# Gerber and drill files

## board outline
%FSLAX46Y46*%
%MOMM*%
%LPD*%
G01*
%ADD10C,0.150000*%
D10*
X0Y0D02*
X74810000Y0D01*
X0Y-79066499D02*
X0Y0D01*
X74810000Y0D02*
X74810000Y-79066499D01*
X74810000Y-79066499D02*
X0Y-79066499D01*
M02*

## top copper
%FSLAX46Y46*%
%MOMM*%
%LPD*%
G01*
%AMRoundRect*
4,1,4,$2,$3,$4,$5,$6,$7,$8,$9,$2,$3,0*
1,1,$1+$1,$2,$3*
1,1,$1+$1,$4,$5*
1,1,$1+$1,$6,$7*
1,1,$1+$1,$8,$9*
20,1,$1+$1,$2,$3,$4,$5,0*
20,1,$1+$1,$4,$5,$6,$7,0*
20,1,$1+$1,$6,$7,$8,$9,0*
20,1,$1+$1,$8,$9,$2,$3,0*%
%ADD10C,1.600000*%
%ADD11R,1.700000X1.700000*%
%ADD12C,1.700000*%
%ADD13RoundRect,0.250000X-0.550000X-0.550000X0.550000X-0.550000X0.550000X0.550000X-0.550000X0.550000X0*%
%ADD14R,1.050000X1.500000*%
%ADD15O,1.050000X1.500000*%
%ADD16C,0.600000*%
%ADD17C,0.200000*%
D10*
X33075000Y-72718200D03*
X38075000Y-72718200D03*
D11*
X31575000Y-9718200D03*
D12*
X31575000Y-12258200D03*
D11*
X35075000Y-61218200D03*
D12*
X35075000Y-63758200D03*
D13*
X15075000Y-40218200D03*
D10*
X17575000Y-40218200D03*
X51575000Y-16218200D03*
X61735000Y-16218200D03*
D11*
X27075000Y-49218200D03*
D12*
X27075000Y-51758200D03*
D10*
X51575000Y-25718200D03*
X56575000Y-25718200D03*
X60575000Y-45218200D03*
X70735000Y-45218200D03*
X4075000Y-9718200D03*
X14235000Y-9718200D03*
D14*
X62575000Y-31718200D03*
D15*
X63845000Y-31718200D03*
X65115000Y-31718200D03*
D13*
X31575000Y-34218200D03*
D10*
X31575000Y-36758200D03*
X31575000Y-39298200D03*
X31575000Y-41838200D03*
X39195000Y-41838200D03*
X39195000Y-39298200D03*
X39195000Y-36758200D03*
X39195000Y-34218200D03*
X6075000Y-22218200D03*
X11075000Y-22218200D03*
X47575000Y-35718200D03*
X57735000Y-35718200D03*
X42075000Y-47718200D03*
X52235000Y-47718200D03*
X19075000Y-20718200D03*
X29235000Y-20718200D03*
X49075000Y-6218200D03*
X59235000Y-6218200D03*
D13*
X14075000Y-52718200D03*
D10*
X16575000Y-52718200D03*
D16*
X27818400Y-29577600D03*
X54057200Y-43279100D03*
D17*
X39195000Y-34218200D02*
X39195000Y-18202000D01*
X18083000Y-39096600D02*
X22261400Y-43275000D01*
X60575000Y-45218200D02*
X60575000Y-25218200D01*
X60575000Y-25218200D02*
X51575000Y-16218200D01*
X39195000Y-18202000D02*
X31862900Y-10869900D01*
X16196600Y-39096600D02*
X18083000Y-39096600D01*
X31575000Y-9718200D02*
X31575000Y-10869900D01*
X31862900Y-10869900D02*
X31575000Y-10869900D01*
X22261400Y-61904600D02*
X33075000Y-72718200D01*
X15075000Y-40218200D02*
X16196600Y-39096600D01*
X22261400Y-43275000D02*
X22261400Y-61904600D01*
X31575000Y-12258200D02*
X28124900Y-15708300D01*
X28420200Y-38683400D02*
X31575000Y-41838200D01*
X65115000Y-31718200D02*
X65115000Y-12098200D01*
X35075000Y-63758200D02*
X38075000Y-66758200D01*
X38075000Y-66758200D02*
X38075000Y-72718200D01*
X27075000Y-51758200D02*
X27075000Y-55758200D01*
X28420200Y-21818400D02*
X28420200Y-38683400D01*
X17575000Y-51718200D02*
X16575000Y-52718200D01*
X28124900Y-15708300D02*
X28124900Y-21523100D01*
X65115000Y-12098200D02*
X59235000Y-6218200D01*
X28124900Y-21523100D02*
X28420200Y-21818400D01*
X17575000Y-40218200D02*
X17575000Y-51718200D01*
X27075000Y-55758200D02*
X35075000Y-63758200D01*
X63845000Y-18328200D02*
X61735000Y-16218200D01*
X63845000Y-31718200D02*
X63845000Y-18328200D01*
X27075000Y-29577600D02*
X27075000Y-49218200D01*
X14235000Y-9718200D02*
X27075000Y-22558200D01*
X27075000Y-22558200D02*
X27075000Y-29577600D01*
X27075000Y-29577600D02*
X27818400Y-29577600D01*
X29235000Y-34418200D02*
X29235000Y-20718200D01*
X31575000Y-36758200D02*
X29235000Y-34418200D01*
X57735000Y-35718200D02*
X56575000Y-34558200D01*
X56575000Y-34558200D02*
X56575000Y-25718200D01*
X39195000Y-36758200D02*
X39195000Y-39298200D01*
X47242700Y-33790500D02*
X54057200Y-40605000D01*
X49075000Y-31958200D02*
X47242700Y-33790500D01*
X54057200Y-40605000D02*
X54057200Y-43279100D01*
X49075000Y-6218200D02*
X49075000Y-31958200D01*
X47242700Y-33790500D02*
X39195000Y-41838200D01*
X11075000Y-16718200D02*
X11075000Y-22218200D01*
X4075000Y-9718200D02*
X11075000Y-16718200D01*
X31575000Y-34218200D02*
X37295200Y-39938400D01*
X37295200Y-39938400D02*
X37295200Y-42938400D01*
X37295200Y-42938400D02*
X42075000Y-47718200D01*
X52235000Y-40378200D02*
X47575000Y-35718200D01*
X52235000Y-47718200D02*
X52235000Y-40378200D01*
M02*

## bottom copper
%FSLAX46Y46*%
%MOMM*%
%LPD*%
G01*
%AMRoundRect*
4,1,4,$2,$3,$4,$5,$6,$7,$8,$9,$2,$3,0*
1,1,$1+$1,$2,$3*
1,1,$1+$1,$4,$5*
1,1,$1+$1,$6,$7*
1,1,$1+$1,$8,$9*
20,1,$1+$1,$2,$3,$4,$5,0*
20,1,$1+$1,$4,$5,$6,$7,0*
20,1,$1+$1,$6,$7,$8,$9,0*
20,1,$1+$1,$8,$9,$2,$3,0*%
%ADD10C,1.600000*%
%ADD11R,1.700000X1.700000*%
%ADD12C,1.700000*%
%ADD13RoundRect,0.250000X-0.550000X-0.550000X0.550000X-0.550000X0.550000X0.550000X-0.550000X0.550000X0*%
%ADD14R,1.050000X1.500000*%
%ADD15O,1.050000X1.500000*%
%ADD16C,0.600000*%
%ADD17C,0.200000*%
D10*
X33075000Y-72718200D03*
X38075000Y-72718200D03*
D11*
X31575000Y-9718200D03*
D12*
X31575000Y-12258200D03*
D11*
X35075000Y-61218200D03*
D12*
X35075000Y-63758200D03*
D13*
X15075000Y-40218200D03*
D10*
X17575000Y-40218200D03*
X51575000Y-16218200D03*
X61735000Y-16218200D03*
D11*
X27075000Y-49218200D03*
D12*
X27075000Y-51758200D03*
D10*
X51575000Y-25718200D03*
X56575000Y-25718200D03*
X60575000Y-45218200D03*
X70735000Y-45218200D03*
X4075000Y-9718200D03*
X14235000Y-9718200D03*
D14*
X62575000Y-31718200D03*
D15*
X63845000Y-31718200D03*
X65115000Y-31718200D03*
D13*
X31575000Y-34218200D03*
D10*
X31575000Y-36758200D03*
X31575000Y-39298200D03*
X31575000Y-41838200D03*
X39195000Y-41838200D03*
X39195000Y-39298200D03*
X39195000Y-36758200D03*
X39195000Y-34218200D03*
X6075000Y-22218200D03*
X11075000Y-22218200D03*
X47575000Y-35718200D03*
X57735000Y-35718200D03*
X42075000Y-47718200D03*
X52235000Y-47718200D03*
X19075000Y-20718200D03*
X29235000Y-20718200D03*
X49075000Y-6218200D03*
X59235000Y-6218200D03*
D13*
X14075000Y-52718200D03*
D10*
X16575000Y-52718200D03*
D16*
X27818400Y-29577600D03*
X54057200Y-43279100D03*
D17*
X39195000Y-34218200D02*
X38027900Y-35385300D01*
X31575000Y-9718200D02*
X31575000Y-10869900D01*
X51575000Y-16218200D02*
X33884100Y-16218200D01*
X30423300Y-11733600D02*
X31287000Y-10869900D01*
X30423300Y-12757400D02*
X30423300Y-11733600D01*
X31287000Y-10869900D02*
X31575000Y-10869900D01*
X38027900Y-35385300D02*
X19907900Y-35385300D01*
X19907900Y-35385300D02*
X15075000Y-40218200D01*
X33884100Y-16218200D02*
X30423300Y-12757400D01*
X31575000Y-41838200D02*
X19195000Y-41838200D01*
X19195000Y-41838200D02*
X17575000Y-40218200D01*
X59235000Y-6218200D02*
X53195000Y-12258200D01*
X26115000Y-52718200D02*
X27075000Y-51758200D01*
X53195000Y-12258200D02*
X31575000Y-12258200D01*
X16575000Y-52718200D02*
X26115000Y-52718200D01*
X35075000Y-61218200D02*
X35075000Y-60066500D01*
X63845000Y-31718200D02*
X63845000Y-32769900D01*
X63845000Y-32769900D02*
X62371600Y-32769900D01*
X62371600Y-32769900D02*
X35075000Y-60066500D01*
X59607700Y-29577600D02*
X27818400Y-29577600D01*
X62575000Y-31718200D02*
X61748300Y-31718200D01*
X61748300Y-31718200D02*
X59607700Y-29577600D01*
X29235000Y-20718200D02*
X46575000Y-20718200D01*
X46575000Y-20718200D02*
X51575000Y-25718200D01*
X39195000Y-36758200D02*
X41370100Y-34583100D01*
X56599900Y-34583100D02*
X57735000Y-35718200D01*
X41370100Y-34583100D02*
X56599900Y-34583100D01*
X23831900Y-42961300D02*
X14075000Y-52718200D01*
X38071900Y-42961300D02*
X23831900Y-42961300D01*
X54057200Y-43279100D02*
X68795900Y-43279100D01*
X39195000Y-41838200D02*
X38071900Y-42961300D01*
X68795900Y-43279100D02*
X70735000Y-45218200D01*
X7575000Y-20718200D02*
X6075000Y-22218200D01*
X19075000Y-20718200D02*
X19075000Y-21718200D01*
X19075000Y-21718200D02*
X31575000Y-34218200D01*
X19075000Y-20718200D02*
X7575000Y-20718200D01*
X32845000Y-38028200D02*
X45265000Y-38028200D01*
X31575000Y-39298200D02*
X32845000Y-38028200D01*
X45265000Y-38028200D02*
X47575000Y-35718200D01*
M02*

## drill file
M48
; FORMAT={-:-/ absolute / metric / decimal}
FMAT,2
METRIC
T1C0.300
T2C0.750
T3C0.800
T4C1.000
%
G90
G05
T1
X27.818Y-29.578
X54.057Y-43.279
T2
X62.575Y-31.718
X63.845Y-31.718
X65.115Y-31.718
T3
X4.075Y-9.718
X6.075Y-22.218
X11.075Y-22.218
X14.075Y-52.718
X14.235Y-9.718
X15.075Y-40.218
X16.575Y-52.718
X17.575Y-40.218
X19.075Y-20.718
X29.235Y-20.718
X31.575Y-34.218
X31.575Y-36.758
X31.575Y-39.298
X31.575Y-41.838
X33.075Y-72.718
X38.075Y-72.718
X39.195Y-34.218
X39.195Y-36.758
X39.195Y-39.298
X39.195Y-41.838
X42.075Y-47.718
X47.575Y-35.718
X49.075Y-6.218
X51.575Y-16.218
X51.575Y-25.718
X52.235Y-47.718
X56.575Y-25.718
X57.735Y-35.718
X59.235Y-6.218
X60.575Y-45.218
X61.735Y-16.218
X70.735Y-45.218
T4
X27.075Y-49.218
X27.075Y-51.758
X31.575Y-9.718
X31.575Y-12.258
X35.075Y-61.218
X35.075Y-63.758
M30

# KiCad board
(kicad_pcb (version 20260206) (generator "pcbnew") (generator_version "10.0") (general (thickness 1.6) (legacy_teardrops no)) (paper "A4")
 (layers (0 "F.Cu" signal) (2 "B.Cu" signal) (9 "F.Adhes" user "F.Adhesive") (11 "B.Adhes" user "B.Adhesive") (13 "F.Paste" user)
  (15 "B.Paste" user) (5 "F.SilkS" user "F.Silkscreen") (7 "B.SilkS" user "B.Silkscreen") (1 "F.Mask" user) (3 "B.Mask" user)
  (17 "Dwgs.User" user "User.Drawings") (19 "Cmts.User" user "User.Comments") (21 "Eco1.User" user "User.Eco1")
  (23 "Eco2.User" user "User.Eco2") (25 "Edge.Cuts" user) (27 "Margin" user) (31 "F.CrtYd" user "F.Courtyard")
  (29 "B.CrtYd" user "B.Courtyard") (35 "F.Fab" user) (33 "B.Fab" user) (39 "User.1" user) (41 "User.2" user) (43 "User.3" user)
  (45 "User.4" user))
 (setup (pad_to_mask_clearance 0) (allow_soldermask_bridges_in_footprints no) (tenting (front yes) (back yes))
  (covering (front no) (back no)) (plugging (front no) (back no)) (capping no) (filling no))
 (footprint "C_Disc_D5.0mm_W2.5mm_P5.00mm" (layer "F.Cu") (at 33.075 72.7182)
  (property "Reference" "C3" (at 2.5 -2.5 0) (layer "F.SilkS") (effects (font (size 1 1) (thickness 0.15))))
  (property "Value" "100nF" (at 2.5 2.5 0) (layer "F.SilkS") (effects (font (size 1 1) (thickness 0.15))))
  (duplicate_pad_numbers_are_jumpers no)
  (pad "1" thru_hole circle (at 0 0) (size 1.6 1.6) (drill 0.8) (layers "*.Cu" "*.Mask") (remove_unused_layers no) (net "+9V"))
  (pad "2" thru_hole circle (at 5 0) (size 1.6 1.6) (drill 0.8) (layers "*.Cu" "*.Mask") (remove_unused_layers no) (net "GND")))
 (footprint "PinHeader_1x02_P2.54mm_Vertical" (layer "F.Cu") (at 31.575 9.7182)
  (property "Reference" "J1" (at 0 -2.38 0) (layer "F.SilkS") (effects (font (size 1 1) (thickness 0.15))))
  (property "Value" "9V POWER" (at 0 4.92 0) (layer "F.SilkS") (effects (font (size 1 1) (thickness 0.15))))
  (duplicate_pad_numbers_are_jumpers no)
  (pad "1" thru_hole rect (at 0 0) (size 1.7 1.7) (drill 1) (layers "*.Cu" "*.Mask") (remove_unused_layers no) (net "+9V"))
  (pad "2" thru_hole circle (at 0 2.54) (size 1.7 1.7) (drill 1) (layers "*.Cu" "*.Mask") (remove_unused_layers no) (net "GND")))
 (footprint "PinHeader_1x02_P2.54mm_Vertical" (layer "F.Cu") (at 35.075 61.2182)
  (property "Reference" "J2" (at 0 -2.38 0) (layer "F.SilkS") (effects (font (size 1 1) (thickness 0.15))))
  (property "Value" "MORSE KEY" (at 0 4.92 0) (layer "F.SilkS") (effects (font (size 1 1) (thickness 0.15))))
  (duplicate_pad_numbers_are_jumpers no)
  (pad "1" thru_hole rect (at 0 0) (size 1.7 1.7) (drill 1) (layers "*.Cu" "*.Mask") (remove_unused_layers no) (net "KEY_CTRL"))
  (pad "2" thru_hole circle (at 0 2.54) (size 1.7 1.7) (drill 1) (layers "*.Cu" "*.Mask") (remove_unused_layers no) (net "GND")))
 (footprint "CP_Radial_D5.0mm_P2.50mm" (layer "F.Cu") (at 15.075 40.2182)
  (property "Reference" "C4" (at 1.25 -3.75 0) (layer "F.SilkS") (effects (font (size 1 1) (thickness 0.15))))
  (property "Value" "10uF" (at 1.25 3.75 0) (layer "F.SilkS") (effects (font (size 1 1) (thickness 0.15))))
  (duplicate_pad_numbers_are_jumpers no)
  (pad "1" thru_hole roundrect (at 0 0) (size 1.6 1.6) (drill 0.8) (layers "*.Cu" "*.Mask") (remove_unused_layers no)
   (roundrect_rratio 0.15625) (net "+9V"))
  (pad "2" thru_hole circle (at 2.5 0) (size 1.6 1.6) (drill 0.8) (layers "*.Cu" "*.Mask") (remove_unused_layers no) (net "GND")))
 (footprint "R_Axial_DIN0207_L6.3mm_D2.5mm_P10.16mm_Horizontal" (layer "F.Cu") (at 51.575 16.2182)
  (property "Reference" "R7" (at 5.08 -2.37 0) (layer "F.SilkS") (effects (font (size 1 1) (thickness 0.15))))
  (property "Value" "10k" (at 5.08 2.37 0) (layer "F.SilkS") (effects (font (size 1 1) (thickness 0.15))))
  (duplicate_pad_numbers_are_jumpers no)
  (pad "1" thru_hole circle (at 0 0) (size 1.6 1.6) (drill 0.8) (layers "*.Cu" "*.Mask") (remove_unused_layers no) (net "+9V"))
  (pad "2" thru_hole circle (at 10.16 0) (size 1.6 1.6) (drill 0.8) (layers "*.Cu" "*.Mask") (remove_unused_layers no) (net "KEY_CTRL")))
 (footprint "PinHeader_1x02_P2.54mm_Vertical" (layer "F.Cu") (at 27.075 49.2182)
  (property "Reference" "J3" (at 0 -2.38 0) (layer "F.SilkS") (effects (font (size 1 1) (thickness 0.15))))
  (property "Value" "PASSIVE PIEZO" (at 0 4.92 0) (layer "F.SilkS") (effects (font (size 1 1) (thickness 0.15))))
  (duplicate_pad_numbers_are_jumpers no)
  (pad "1" thru_hole rect (at 0 0) (size 1.7 1.7) (drill 1) (layers "*.Cu" "*.Mask") (remove_unused_layers no) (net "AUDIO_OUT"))
  (pad "2" thru_hole circle (at 0 2.54) (size 1.7 1.7) (drill 1) (layers "*.Cu" "*.Mask") (remove_unused_layers no) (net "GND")))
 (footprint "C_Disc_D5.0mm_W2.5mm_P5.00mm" (layer "F.Cu") (at 51.575 25.7182)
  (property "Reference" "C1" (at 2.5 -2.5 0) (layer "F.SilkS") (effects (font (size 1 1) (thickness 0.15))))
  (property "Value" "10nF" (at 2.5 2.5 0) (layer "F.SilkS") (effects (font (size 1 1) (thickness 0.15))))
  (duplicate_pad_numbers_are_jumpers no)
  (pad "1" thru_hole circle (at 0 0) (size 1.6 1.6) (drill 0.8) (layers "*.Cu" "*.Mask") (remove_unused_layers no) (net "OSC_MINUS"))
  (pad "2" thru_hole circle (at 5 0) (size 1.6 1.6) (drill 0.8) (layers "*.Cu" "*.Mask") (remove_unused_layers no) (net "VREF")))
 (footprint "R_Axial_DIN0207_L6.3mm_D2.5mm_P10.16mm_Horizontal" (layer "F.Cu") (at 60.575 45.2182)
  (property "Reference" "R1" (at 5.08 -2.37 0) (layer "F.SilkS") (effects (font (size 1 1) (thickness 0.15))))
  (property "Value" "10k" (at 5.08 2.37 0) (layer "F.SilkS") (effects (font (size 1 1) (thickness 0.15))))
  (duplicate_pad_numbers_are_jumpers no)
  (pad "1" thru_hole circle (at 0 0) (size 1.6 1.6) (drill 0.8) (layers "*.Cu" "*.Mask") (remove_unused_layers no) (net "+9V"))
  (pad "2" thru_hole circle (at 10.16 0) (size 1.6 1.6) (drill 0.8) (layers "*.Cu" "*.Mask") (remove_unused_layers no) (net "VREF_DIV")))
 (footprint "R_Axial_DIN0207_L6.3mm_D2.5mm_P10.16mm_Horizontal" (layer "F.Cu") (at 4.075 9.7182)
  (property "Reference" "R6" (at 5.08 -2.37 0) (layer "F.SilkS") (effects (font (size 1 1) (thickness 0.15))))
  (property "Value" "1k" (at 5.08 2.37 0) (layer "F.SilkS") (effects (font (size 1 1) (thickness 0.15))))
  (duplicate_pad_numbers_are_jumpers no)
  (pad "1" thru_hole circle (at 0 0) (size 1.6 1.6) (drill 0.8) (layers "*.Cu" "*.Mask") (remove_unused_layers no) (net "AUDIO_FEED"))
  (pad "2" thru_hole circle (at 10.16 0) (size 1.6 1.6) (drill 0.8) (layers "*.Cu" "*.Mask") (remove_unused_layers no) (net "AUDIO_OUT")))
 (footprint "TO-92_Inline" (layer "F.Cu") (at 62.575 31.7182)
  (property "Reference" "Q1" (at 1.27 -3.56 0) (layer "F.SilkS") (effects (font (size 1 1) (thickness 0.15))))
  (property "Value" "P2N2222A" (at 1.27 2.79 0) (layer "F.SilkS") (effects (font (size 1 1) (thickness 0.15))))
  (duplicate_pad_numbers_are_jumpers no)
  (pad "1" thru_hole rect (at 0 0) (size 1.05 1.5) (drill 0.75) (layers "*.Cu" "*.Mask") (remove_unused_layers no) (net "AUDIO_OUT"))
  (pad "2" thru_hole oval (at 1.27 0) (size 1.05 1.5) (drill 0.75) (layers "*.Cu" "*.Mask") (remove_unused_layers no) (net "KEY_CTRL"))
  (pad "3" thru_hole oval (at 2.54 0) (size 1.05 1.5) (drill 0.75) (layers "*.Cu" "*.Mask") (remove_unused_layers no) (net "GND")))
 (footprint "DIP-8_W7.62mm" (layer "F.Cu") (at 31.575 34.2182)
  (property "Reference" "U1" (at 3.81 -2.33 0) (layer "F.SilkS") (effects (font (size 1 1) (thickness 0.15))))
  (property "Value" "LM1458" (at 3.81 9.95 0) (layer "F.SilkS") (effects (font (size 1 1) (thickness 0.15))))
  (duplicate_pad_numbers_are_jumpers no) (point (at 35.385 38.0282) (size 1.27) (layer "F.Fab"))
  (pad "1" thru_hole roundrect (at 0 0) (size 1.6 1.6) (drill 0.8) (layers "*.Cu" "*.Mask") (remove_unused_layers no)
   (roundrect_rratio 0.15625) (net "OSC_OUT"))
  (pad "2" thru_hole circle (at 0 2.54) (size 1.6 1.6) (drill 0.8) (layers "*.Cu" "*.Mask") (remove_unused_layers no) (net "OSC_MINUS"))
  (pad "3" thru_hole circle (at 0 5.08) (size 1.6 1.6) (drill 0.8) (layers "*.Cu" "*.Mask") (remove_unused_layers no) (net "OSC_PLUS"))
  (pad "4" thru_hole circle (at 0 7.62) (size 1.6 1.6) (drill 0.8) (layers "*.Cu" "*.Mask") (remove_unused_layers no) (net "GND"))
  (pad "5" thru_hole circle (at 7.62 7.62) (size 1.6 1.6) (drill 0.8) (layers "*.Cu" "*.Mask") (remove_unused_layers no) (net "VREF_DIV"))
  (pad "6" thru_hole circle (at 7.62 5.08) (size 1.6 1.6) (drill 0.8) (layers "*.Cu" "*.Mask") (remove_unused_layers no) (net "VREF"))
  (pad "7" thru_hole circle (at 7.62 2.54) (size 1.6 1.6) (drill 0.8) (layers "*.Cu" "*.Mask") (remove_unused_layers no) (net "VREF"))
  (pad "8" thru_hole circle (at 7.62 0) (size 1.6 1.6) (drill 0.8) (layers "*.Cu" "*.Mask") (remove_unused_layers no) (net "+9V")))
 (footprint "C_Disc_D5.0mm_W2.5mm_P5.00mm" (layer "F.Cu") (at 6.075 22.2182)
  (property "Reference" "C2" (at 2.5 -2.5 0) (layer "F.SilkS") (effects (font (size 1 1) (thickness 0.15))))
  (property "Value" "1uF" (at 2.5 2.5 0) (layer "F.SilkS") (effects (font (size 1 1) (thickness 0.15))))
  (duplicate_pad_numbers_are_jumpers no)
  (pad "1" thru_hole circle (at 0 0) (size 1.6 1.6) (drill 0.8) (layers "*.Cu" "*.Mask") (remove_unused_layers no) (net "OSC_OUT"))
  (pad "2" thru_hole circle (at 5 0) (size 1.6 1.6) (drill 0.8) (layers "*.Cu" "*.Mask") (remove_unused_layers no) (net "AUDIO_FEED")))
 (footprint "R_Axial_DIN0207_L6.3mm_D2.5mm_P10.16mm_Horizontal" (layer "F.Cu") (at 47.575 35.7182)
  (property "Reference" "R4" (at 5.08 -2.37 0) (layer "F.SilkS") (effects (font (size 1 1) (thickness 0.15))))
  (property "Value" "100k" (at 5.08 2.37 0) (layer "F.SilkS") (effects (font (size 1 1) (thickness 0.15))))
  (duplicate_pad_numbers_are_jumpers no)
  (pad "1" thru_hole circle (at 0 0) (size 1.6 1.6) (drill 0.8) (layers "*.Cu" "*.Mask") (remove_unused_layers no) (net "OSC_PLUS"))
  (pad "2" thru_hole circle (at 10.16 0) (size 1.6 1.6) (drill 0.8) (layers "*.Cu" "*.Mask") (remove_unused_layers no) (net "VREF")))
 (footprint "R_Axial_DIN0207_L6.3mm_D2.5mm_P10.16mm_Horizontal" (layer "F.Cu") (at 42.075 47.7182)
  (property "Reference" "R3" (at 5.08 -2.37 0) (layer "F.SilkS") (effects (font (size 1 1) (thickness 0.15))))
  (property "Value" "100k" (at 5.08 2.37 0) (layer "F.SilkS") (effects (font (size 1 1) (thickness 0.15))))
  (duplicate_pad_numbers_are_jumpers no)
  (pad "1" thru_hole circle (at 0 0) (size 1.6 1.6) (drill 0.8) (layers "*.Cu" "*.Mask") (remove_unused_layers no) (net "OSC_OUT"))
  (pad "2" thru_hole circle (at 10.16 0) (size 1.6 1.6) (drill 0.8) (layers "*.Cu" "*.Mask") (remove_unused_layers no) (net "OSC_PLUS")))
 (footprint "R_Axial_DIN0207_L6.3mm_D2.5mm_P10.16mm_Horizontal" (layer "F.Cu") (at 19.075 20.7182)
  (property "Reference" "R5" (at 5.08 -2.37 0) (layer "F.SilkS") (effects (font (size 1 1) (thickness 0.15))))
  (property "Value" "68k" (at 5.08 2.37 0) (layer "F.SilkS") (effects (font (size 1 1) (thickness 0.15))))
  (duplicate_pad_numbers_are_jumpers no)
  (pad "1" thru_hole circle (at 0 0) (size 1.6 1.6) (drill 0.8) (layers "*.Cu" "*.Mask") (remove_unused_layers no) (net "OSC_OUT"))
  (pad "2" thru_hole circle (at 10.16 0) (size 1.6 1.6) (drill 0.8) (layers "*.Cu" "*.Mask") (remove_unused_layers no) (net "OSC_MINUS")))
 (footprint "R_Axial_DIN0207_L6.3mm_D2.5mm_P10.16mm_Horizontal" (layer "F.Cu") (at 49.075 6.2182)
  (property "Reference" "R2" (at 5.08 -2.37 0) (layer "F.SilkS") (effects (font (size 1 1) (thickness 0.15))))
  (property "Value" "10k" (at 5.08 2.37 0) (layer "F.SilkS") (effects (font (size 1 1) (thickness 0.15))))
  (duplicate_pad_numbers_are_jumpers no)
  (pad "1" thru_hole circle (at 0 0) (size 1.6 1.6) (drill 0.8) (layers "*.Cu" "*.Mask") (remove_unused_layers no) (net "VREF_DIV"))
  (pad "2" thru_hole circle (at 10.16 0) (size 1.6 1.6) (drill 0.8) (layers "*.Cu" "*.Mask") (remove_unused_layers no) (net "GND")))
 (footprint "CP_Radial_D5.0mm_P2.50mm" (layer "F.Cu") (at 14.075 52.7182)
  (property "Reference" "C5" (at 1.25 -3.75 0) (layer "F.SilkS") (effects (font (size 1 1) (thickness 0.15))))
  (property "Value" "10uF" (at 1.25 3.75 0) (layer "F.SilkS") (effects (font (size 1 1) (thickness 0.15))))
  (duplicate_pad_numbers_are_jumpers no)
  (pad "1" thru_hole roundrect (at 0 0) (size 1.6 1.6) (drill 0.8) (layers "*.Cu" "*.Mask") (remove_unused_layers no)
   (roundrect_rratio 0.15625) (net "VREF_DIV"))
  (pad "2" thru_hole circle (at 2.5 0) (size 1.6 1.6) (drill 0.8) (layers "*.Cu" "*.Mask") (remove_unused_layers no) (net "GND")))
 (gr_line (start 0 0) (end 74.81 0) (stroke (width 0.15) (type default)) (layer "Edge.Cuts"))
 (gr_line (start 0 79.066499) (end 0 0) (stroke (width 0.15) (type default)) (layer "Edge.Cuts"))
 (gr_line (start 74.81 0) (end 74.81 79.066499) (stroke (width 0.15) (type default)) (layer "Edge.Cuts"))
 (gr_line (start 74.81 79.066499) (end 0 79.066499) (stroke (width 0.15) (type default)) (layer "Edge.Cuts"))
 (segment (start 39.195 34.2182) (end 39.195 18.202) (width 0.2) (layer "F.Cu") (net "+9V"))
 (segment (start 18.083 39.0966) (end 22.2614 43.275) (width 0.2) (layer "F.Cu") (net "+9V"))
 (segment (start 60.575 45.2182) (end 60.575 25.2182) (width 0.2) (layer "F.Cu") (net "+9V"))
 (segment (start 60.575 25.2182) (end 51.575 16.2182) (width 0.2) (layer "F.Cu") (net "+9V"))
 (segment (start 39.195 18.202) (end 31.8629 10.8699) (width 0.2) (layer "F.Cu") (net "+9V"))
 (segment (start 16.1966 39.0966) (end 18.083 39.0966) (width 0.2) (layer "F.Cu") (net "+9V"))
 (segment (start 31.575 9.7182) (end 31.575 10.8699) (width 0.2) (layer "F.Cu") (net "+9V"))
 (segment (start 31.8629 10.8699) (end 31.575 10.8699) (width 0.2) (layer "F.Cu") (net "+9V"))
 (segment (start 22.2614 61.9046) (end 33.075 72.7182) (width 0.2) (layer "F.Cu") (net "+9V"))
 (segment (start 15.075 40.2182) (end 16.1966 39.0966) (width 0.2) (layer "F.Cu") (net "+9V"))
 (segment (start 22.2614 43.275) (end 22.2614 61.9046) (width 0.2) (layer "F.Cu") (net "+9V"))
 (segment (start 39.195 34.2182) (end 38.0279 35.3853) (width 0.2) (layer "B.Cu") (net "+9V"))
 (segment (start 31.575 9.7182) (end 31.575 10.8699) (width 0.2) (layer "B.Cu") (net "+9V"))
 (segment (start 51.575 16.2182) (end 33.8841 16.2182) (width 0.2) (layer "B.Cu") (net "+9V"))
 (segment (start 30.4233 11.7336) (end 31.287 10.8699) (width 0.2) (layer "B.Cu") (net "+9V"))
 (segment (start 30.4233 12.7574) (end 30.4233 11.7336) (width 0.2) (layer "B.Cu") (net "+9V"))
 (segment (start 31.287 10.8699) (end 31.575 10.8699) (width 0.2) (layer "B.Cu") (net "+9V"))
 (segment (start 38.0279 35.3853) (end 19.9079 35.3853) (width 0.2) (layer "B.Cu") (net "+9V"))
 (segment (start 19.9079 35.3853) (end 15.075 40.2182) (width 0.2) (layer "B.Cu") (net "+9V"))
 (segment (start 33.8841 16.2182) (end 30.4233 12.7574) (width 0.2) (layer "B.Cu") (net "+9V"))
 (segment (start 31.575 12.2582) (end 28.1249 15.7083) (width 0.2) (layer "F.Cu") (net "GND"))
 (segment (start 28.4202 38.6834) (end 31.575 41.8382) (width 0.2) (layer "F.Cu") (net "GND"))
 (segment (start 65.115 31.7182) (end 65.115 12.0982) (width 0.2) (layer "F.Cu") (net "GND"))
 (segment (start 35.075 63.7582) (end 38.075 66.7582) (width 0.2) (layer "F.Cu") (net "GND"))
 (segment (start 38.075 66.7582) (end 38.075 72.7182) (width 0.2) (layer "F.Cu") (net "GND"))
 (segment (start 27.075 51.7582) (end 27.075 55.7582) (width 0.2) (layer "F.Cu") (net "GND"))
 (segment (start 28.4202 21.8184) (end 28.4202 38.6834) (width 0.2) (layer "F.Cu") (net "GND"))
 (segment (start 17.575 51.7182) (end 16.575 52.7182) (width 0.2) (layer "F.Cu") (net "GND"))
 (segment (start 28.1249 15.7083) (end 28.1249 21.5231) (width 0.2) (layer "F.Cu") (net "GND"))
 (segment (start 65.115 12.0982) (end 59.235 6.2182) (width 0.2) (layer "F.Cu") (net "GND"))
 (segment (start 28.1249 21.5231) (end 28.4202 21.8184) (width 0.2) (layer "F.Cu") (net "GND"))
 (segment (start 17.575 40.2182) (end 17.575 51.7182) (width 0.2) (layer "F.Cu") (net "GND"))
 (segment (start 27.075 55.7582) (end 35.075 63.7582) (width 0.2) (layer "F.Cu") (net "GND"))
 (segment (start 31.575 41.8382) (end 19.195 41.8382) (width 0.2) (layer "B.Cu") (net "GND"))
 (segment (start 19.195 41.8382) (end 17.575 40.2182) (width 0.2) (layer "B.Cu") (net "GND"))
 (segment (start 59.235 6.2182) (end 53.195 12.2582) (width 0.2) (layer "B.Cu") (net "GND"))
 (segment (start 26.115 52.7182) (end 27.075 51.7582) (width 0.2) (layer "B.Cu") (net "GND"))
 (segment (start 53.195 12.2582) (end 31.575 12.2582) (width 0.2) (layer "B.Cu") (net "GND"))
 (segment (start 16.575 52.7182) (end 26.115 52.7182) (width 0.2) (layer "B.Cu") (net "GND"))
 (segment (start 63.845 18.3282) (end 61.735 16.2182) (width 0.2) (layer "F.Cu") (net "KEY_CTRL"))
 (segment (start 63.845 31.7182) (end 63.845 18.3282) (width 0.2) (layer "F.Cu") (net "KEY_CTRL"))
 (segment (start 35.075 61.2182) (end 35.075 60.0665) (width 0.2) (layer "B.Cu") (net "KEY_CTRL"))
 (segment (start 63.845 31.7182) (end 63.845 32.7699) (width 0.2) (layer "B.Cu") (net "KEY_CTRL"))
 (segment (start 63.845 32.7699) (end 62.3716 32.7699) (width 0.2) (layer "B.Cu") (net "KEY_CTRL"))
 (segment (start 62.3716 32.7699) (end 35.075 60.0665) (width 0.2) (layer "B.Cu") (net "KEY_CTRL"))
 (segment (start 27.075 29.5776) (end 27.075 49.2182) (width 0.2) (layer "F.Cu") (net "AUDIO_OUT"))
 (segment (start 14.235 9.7182) (end 27.075 22.5582) (width 0.2) (layer "F.Cu") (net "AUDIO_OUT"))
 (segment (start 27.075 22.5582) (end 27.075 29.5776) (width 0.2) (layer "F.Cu") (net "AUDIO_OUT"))
 (segment (start 27.075 29.5776) (end 27.8184 29.5776) (width 0.2) (layer "F.Cu") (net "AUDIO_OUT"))
 (via (at 27.8184 29.5776) (size 0.6) (drill 0.3) (layers "F.Cu" "B.Cu") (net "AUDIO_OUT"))
 (segment (start 59.6077 29.5776) (end 27.8184 29.5776) (width 0.2) (layer "B.Cu") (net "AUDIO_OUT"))
 (segment (start 62.575 31.7182) (end 61.7483 31.7182) (width 0.2) (layer "B.Cu") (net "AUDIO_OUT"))
 (segment (start 61.7483 31.7182) (end 59.6077 29.5776) (width 0.2) (layer "B.Cu") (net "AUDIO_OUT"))
 (segment (start 29.235 34.4182) (end 29.235 20.7182) (width 0.2) (layer "F.Cu") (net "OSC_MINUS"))
 (segment (start 31.575 36.7582) (end 29.235 34.4182) (width 0.2) (layer "F.Cu") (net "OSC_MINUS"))
 (segment (start 29.235 20.7182) (end 46.575 20.7182) (width 0.2) (layer "B.Cu") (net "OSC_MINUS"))
 (segment (start 46.575 20.7182) (end 51.575 25.7182) (width 0.2) (layer "B.Cu") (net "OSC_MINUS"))
 (segment (start 57.735 35.7182) (end 56.575 34.5582) (width 0.2) (layer "F.Cu") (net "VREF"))
 (segment (start 56.575 34.5582) (end 56.575 25.7182) (width 0.2) (layer "F.Cu") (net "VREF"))
 (segment (start 39.195 36.7582) (end 39.195 39.2982) (width 0.2) (layer "F.Cu") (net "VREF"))
 (segment (start 39.195 36.7582) (end 41.3701 34.5831) (width 0.2) (layer "B.Cu") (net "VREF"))
 (segment (start 56.5999 34.5831) (end 57.735 35.7182) (width 0.2) (layer "B.Cu") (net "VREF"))
 (segment (start 41.3701 34.5831) (end 56.5999 34.5831) (width 0.2) (layer "B.Cu") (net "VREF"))
 (segment (start 47.2427 33.7905) (end 54.0572 40.605) (width 0.2) (layer "F.Cu") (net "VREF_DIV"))
 (segment (start 49.075 31.9582) (end 47.2427 33.7905) (width 0.2) (layer "F.Cu") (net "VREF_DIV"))
 (segment (start 54.0572 40.605) (end 54.0572 43.2791) (width 0.2) (layer "F.Cu") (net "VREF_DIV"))
 (segment (start 49.075 6.2182) (end 49.075 31.9582) (width 0.2) (layer "F.Cu") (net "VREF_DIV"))
 (segment (start 47.2427 33.7905) (end 39.195 41.8382) (width 0.2) (layer "F.Cu") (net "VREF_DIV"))
 (via (at 54.0572 43.2791) (size 0.6) (drill 0.3) (layers "F.Cu" "B.Cu") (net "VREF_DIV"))
 (segment (start 23.8319 42.9613) (end 14.075 52.7182) (width 0.2) (layer "B.Cu") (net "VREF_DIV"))
 (segment (start 38.0719 42.9613) (end 23.8319 42.9613) (width 0.2) (layer "B.Cu") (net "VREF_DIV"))
 (segment (start 54.0572 43.2791) (end 68.7959 43.2791) (width 0.2) (layer "B.Cu") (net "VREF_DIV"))
 (segment (start 39.195 41.8382) (end 38.0719 42.9613) (width 0.2) (layer "B.Cu") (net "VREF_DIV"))
 (segment (start 68.7959 43.2791) (end 70.735 45.2182) (width 0.2) (layer "B.Cu") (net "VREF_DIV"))
 (segment (start 11.075 16.7182) (end 11.075 22.2182) (width 0.2) (layer "F.Cu") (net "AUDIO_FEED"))
 (segment (start 4.075 9.7182) (end 11.075 16.7182) (width 0.2) (layer "F.Cu") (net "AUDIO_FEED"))
 (segment (start 31.575 34.2182) (end 37.2952 39.9384) (width 0.2) (layer "F.Cu") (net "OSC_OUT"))
 (segment (start 37.2952 39.9384) (end 37.2952 42.9384) (width 0.2) (layer "F.Cu") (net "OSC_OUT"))
 (segment (start 37.2952 42.9384) (end 42.075 47.7182) (width 0.2) (layer "F.Cu") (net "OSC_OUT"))
 (segment (start 7.575 20.7182) (end 6.075 22.2182) (width 0.2) (layer "B.Cu") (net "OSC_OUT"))
 (segment (start 19.075 20.7182) (end 19.075 21.7182) (width 0.2) (layer "B.Cu") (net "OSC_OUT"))
 (segment (start 19.075 21.7182) (end 31.575 34.2182) (width 0.2) (layer "B.Cu") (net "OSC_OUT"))
 (segment (start 19.075 20.7182) (end 7.575 20.7182) (width 0.2) (layer "B.Cu") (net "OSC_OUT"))
 (segment (start 52.235 40.3782) (end 47.575 35.7182) (width 0.2) (layer "F.Cu") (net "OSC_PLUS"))
 (segment (start 52.235 47.7182) (end 52.235 40.3782) (width 0.2) (layer "F.Cu") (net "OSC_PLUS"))
 (segment (start 32.845 38.0282) (end 45.265 38.0282) (width 0.2) (layer "B.Cu") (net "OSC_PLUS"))
 (segment (start 31.575 39.2982) (end 32.845 38.0282) (width 0.2) (layer "B.Cu") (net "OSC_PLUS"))
 (segment (start 45.265 38.0282) (end 47.575 35.7182) (width 0.2) (layer "B.Cu") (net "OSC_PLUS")))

